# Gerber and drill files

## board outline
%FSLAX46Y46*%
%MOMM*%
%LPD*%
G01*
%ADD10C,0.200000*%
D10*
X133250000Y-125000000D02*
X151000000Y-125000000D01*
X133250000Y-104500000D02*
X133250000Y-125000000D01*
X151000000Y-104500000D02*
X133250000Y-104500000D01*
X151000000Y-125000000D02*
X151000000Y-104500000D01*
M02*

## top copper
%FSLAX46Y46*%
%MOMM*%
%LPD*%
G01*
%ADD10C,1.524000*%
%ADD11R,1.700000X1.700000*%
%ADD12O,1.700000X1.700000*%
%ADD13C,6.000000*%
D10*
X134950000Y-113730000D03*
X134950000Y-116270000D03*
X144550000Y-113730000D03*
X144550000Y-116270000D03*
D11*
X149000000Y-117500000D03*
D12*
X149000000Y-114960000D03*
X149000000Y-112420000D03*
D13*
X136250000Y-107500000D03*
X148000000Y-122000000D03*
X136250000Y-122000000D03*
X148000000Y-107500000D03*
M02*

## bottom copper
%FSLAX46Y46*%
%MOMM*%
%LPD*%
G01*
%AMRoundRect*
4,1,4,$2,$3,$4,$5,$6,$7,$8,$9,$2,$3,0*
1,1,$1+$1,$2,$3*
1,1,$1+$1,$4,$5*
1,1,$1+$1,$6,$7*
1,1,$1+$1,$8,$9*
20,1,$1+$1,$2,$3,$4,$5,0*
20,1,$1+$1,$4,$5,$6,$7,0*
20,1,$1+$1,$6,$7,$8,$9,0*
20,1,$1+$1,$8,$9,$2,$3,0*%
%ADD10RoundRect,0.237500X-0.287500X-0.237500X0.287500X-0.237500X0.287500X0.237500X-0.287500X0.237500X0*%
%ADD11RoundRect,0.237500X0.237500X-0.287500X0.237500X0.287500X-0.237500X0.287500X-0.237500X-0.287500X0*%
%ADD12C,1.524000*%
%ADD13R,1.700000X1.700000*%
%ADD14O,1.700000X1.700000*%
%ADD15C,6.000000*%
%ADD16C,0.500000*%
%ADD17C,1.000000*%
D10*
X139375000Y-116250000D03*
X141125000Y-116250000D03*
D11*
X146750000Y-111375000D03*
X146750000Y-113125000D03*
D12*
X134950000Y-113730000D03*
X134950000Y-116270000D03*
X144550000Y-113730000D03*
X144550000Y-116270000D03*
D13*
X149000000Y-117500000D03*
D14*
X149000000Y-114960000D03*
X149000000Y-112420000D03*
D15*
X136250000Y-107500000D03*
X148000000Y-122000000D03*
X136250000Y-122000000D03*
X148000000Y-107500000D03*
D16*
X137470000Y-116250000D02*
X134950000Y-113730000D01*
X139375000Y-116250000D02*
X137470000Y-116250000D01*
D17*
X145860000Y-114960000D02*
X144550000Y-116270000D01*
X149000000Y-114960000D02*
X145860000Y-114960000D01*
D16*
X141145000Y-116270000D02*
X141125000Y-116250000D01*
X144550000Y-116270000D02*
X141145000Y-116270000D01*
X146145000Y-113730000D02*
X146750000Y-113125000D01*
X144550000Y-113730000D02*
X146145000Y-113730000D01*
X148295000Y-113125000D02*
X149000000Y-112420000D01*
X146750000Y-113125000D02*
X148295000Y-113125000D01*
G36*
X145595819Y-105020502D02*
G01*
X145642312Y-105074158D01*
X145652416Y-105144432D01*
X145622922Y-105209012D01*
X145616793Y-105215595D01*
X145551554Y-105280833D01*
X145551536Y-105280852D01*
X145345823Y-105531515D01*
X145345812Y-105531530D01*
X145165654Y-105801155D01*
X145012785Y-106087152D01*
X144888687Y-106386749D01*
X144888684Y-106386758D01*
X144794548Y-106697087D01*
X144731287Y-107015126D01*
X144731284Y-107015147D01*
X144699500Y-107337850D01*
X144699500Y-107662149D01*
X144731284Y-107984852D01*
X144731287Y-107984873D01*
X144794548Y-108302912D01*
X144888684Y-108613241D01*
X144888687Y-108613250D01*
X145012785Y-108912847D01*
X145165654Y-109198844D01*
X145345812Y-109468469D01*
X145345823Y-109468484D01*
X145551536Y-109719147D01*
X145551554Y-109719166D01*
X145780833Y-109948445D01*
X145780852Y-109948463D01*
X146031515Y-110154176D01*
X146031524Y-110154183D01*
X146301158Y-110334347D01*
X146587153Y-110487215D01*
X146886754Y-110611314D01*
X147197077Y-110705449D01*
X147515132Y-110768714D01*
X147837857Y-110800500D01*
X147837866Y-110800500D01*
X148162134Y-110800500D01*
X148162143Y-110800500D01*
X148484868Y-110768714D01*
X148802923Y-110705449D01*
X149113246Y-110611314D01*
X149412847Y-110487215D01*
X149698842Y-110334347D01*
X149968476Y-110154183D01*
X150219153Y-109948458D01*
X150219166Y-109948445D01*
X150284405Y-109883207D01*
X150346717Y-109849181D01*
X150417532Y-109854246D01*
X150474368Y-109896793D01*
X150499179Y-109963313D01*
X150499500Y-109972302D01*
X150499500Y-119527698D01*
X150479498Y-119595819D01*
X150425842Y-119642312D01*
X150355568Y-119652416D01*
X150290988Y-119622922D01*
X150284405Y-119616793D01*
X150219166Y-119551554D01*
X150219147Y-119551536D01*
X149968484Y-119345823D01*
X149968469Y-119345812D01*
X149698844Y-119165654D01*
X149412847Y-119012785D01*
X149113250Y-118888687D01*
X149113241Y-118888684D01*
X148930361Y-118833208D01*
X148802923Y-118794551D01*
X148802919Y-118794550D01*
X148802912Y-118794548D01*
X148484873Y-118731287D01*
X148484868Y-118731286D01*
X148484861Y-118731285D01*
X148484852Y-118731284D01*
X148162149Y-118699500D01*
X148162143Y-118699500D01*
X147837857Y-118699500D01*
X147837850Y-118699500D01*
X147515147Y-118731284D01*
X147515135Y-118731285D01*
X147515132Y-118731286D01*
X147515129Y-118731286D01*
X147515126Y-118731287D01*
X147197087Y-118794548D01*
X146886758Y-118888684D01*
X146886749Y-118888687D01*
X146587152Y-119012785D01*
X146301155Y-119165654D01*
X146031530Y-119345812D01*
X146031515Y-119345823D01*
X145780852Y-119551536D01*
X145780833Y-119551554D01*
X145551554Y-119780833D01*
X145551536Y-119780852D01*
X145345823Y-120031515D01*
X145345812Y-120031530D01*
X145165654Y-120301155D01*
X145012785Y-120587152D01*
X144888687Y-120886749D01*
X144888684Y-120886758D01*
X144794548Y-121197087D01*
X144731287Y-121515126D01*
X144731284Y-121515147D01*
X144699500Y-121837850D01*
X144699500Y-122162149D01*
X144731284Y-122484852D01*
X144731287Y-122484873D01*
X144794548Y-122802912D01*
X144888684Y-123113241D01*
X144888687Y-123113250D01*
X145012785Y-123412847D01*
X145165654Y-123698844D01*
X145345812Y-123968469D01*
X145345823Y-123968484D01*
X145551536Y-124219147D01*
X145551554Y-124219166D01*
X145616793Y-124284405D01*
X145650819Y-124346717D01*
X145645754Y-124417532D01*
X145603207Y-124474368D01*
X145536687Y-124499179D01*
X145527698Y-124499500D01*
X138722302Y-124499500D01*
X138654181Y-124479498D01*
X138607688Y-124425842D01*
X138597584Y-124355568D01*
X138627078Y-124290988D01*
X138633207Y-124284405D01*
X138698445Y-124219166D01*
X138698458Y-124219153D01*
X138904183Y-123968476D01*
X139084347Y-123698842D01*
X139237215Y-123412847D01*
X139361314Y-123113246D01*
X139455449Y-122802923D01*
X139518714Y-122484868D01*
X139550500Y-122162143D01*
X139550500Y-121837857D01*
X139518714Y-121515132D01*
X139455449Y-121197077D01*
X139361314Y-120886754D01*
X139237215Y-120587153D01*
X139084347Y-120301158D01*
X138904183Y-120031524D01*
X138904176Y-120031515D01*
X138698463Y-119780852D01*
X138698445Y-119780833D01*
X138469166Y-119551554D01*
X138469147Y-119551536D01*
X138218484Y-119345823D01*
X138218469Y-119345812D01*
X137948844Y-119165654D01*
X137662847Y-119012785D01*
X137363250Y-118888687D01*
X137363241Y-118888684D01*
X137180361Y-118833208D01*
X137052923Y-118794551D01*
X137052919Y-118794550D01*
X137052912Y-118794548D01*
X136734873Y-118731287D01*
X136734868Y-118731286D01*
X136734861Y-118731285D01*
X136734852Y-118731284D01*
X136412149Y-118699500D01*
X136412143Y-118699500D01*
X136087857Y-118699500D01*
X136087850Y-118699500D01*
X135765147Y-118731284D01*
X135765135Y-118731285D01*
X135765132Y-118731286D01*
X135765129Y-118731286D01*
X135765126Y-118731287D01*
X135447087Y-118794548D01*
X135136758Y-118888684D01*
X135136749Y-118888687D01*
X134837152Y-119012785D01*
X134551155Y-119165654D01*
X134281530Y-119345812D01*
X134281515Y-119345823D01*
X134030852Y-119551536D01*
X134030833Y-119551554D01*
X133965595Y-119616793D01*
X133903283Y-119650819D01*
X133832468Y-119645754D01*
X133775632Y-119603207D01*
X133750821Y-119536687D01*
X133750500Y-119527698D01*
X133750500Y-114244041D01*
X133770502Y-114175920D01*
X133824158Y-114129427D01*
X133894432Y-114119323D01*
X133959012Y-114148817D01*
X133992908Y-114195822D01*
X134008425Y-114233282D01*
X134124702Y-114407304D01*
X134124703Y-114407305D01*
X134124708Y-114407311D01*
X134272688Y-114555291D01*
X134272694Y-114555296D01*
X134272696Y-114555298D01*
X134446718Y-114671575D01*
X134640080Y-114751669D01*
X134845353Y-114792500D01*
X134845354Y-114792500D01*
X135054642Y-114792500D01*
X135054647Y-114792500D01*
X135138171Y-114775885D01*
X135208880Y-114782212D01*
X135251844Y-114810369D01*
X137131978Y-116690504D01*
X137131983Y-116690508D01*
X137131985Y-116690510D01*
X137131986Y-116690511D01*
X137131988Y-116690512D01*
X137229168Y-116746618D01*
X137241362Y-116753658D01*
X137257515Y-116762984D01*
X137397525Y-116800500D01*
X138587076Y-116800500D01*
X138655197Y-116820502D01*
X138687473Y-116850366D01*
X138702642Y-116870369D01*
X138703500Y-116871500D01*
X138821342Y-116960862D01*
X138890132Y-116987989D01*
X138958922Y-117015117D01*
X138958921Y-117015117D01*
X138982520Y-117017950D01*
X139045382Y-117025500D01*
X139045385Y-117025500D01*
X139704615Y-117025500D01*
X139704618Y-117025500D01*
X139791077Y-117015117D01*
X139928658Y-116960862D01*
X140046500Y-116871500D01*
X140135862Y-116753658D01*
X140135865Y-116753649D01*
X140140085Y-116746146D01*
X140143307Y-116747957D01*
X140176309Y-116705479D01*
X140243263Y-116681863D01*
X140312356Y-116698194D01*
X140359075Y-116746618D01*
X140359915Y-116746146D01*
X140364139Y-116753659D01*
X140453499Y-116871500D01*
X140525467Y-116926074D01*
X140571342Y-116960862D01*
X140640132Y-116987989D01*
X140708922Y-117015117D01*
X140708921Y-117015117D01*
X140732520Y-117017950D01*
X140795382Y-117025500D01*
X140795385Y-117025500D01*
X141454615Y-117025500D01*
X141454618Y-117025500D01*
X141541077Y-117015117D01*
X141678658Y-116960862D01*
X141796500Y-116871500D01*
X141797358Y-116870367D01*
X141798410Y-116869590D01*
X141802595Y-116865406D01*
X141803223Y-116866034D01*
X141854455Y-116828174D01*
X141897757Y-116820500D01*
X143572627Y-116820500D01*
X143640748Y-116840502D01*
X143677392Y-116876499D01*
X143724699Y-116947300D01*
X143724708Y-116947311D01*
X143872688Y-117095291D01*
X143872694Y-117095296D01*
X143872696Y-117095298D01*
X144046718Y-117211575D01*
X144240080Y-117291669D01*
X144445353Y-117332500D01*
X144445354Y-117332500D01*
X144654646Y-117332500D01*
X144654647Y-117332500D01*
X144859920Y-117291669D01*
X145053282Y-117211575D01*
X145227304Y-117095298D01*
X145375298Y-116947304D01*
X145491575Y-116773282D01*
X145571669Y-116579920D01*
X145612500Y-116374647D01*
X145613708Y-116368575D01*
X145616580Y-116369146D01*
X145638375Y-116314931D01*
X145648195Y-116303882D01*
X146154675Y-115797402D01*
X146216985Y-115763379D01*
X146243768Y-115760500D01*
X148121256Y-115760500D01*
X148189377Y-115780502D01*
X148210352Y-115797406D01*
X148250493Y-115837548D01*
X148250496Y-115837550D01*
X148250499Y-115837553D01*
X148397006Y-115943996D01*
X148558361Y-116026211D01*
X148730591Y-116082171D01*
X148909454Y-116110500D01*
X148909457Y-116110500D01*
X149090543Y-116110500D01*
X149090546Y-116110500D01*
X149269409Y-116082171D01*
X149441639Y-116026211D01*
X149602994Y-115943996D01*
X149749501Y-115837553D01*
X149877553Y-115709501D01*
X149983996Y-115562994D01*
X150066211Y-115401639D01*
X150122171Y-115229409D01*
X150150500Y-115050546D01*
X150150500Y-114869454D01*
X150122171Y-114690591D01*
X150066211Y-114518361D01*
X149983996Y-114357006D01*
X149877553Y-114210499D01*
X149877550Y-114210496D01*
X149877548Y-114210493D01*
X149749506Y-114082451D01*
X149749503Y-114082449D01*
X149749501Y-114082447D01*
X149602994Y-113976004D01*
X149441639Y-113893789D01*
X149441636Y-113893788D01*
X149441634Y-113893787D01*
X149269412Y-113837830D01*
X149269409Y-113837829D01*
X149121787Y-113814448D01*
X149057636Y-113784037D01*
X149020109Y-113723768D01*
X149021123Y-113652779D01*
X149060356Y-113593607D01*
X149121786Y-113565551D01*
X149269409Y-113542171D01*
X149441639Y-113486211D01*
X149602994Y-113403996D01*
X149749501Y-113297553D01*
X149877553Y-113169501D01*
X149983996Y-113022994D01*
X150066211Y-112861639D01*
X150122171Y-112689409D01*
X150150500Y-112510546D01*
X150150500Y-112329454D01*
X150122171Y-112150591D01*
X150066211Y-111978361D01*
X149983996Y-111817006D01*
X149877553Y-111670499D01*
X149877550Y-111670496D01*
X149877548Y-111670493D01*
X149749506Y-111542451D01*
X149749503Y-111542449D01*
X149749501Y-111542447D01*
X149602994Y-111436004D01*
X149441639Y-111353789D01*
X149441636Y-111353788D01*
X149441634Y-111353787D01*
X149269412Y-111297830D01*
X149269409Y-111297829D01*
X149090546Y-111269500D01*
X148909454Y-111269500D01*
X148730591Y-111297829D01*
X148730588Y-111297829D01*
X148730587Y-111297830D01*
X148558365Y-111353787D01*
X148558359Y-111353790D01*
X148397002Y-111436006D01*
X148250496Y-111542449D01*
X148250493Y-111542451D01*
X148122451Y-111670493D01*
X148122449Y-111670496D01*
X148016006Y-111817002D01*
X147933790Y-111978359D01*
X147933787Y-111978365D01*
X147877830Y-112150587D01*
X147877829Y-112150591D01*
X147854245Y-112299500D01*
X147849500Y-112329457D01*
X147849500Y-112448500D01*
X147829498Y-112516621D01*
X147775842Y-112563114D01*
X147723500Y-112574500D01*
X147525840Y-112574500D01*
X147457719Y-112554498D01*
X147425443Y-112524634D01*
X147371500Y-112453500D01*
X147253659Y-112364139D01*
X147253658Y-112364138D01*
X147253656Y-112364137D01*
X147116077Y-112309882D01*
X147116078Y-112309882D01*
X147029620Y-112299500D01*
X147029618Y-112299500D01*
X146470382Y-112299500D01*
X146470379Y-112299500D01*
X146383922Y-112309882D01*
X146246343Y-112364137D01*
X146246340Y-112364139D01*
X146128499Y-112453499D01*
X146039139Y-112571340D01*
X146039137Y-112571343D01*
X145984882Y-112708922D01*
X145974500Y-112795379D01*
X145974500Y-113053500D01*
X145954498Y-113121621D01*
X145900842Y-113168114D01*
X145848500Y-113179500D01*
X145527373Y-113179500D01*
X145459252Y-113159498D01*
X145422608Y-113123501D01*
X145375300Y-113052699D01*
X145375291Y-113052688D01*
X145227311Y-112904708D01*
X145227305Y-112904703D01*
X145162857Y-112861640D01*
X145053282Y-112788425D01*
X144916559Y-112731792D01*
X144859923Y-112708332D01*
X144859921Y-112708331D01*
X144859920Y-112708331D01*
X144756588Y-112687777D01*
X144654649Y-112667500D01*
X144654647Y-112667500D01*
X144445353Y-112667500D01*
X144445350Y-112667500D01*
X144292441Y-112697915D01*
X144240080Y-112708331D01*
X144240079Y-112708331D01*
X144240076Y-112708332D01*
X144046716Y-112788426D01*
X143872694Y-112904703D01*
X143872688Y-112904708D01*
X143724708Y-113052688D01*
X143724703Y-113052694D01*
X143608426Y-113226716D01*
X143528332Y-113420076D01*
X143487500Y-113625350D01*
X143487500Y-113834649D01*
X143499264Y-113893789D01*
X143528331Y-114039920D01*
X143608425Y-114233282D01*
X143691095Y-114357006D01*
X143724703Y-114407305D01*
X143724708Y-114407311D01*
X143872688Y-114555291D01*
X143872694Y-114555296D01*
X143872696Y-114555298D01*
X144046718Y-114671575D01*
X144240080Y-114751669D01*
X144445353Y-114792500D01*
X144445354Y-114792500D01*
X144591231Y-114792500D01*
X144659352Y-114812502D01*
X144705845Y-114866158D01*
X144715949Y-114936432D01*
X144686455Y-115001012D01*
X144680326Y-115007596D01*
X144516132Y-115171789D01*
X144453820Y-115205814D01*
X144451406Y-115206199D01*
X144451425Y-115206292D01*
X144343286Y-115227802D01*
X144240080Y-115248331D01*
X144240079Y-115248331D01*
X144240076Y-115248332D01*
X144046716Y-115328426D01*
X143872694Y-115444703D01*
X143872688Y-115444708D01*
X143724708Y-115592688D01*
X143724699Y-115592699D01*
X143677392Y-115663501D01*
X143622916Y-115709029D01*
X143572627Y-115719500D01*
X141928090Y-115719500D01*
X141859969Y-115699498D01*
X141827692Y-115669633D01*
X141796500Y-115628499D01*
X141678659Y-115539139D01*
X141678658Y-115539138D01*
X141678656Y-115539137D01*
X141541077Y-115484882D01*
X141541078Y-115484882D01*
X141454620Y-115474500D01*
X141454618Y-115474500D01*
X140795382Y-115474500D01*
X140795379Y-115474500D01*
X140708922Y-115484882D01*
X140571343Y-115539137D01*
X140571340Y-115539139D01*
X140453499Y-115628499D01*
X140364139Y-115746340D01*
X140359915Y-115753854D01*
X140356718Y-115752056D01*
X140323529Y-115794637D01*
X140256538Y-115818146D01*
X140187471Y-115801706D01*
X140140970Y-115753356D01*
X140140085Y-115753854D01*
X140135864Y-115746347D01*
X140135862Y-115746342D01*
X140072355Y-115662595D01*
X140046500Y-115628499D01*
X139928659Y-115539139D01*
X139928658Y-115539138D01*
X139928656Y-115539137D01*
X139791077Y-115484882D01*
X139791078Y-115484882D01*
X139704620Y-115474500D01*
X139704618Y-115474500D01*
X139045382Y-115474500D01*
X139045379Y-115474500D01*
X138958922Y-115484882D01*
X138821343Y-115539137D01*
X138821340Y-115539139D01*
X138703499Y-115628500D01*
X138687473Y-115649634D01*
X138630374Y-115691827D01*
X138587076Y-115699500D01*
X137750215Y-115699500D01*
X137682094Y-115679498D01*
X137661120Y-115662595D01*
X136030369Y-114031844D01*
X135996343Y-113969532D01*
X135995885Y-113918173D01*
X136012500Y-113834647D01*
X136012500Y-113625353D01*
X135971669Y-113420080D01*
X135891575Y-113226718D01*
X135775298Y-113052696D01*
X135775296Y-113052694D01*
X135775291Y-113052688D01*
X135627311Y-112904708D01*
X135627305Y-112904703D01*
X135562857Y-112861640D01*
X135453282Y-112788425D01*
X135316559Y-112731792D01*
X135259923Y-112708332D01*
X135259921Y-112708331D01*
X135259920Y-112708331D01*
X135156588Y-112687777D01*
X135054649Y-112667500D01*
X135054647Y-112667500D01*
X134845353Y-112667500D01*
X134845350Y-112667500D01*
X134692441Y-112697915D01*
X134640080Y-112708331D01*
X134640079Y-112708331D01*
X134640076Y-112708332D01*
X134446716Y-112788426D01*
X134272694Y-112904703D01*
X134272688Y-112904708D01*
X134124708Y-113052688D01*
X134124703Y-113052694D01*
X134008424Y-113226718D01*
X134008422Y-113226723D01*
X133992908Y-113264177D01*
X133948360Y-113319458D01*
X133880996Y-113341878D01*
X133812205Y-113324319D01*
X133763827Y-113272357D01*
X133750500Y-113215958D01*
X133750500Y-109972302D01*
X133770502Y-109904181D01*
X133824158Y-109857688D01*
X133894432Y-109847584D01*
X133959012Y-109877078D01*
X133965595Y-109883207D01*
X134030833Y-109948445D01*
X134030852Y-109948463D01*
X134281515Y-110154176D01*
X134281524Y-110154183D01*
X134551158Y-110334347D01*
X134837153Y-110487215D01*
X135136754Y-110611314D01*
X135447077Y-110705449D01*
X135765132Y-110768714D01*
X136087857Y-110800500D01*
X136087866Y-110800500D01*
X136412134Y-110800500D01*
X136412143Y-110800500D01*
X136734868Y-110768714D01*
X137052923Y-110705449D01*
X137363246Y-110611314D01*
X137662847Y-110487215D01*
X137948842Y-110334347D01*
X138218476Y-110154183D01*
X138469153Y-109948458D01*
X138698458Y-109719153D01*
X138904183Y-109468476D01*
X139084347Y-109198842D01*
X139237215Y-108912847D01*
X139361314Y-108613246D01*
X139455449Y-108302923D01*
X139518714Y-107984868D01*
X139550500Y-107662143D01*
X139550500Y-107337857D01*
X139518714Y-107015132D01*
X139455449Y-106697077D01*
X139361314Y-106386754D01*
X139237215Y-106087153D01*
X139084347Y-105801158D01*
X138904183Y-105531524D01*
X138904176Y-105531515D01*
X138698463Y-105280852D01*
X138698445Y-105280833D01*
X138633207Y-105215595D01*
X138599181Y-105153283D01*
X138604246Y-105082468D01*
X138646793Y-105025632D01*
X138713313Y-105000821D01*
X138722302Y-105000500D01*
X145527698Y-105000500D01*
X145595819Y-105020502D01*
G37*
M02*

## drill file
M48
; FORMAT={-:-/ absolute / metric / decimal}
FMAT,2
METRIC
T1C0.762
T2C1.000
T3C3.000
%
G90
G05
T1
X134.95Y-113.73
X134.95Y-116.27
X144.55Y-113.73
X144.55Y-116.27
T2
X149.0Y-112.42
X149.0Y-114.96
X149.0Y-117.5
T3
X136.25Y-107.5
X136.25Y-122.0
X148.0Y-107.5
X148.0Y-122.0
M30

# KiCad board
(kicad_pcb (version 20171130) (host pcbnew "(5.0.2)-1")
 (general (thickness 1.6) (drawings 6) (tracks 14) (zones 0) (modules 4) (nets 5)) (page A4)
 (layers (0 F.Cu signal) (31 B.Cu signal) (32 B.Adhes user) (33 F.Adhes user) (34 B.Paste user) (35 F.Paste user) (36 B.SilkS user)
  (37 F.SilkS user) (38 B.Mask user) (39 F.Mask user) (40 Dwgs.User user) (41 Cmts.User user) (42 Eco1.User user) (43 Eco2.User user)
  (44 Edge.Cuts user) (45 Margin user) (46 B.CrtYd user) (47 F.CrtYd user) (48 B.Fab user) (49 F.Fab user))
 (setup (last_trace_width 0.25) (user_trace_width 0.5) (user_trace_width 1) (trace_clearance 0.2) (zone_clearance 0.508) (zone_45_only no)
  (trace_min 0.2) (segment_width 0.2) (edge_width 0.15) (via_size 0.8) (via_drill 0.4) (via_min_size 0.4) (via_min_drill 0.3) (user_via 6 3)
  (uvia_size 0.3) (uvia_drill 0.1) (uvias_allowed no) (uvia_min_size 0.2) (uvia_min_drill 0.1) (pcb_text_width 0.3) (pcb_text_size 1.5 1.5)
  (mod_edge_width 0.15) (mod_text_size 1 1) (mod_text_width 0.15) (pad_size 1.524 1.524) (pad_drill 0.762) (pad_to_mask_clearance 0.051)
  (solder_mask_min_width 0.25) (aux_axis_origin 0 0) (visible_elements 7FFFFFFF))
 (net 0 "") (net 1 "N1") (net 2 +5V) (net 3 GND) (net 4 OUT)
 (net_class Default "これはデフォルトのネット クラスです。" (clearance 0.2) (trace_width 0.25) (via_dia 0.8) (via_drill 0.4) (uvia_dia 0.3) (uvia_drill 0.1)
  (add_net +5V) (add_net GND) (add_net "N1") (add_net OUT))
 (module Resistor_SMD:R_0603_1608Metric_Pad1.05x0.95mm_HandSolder (layer B.Cu) (at 140.25 116.25)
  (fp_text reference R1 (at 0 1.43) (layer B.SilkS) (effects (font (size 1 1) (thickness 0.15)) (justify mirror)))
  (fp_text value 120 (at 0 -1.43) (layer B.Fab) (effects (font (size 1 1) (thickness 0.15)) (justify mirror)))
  (pad 1 smd roundrect (at -0.875 0) (size 1.05 0.95) (layers B.Cu B.Paste B.Mask) (roundrect_rratio 0.25) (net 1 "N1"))
  (pad 2 smd roundrect (at 0.875 0) (size 1.05 0.95) (layers B.Cu B.Paste B.Mask) (roundrect_rratio 0.25) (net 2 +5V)))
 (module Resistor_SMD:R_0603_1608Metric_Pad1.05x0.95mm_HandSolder (layer B.Cu) (at 146.75 112.25 90)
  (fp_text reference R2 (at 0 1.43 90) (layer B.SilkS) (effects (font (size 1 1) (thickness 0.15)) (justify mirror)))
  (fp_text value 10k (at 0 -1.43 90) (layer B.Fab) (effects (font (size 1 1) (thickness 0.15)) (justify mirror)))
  (pad 2 smd roundrect (at 0.875 0 90) (size 1.05 0.95) (layers B.Cu B.Paste B.Mask) (roundrect_rratio 0.25) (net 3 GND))
  (pad 1 smd roundrect (at -0.875 0 90) (size 1.05 0.95) (layers B.Cu B.Paste B.Mask) (roundrect_rratio 0.25) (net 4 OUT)))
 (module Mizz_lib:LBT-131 (layer F.Cu) (at 139.75 115)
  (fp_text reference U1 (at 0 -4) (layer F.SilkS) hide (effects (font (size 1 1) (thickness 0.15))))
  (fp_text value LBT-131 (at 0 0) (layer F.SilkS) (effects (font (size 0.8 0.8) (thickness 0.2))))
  (pad 1 thru_hole circle (at -4.8 -1.27) (size 1.524 1.524) (drill 0.762) (layers *.Cu *.Mask) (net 1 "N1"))
  (pad 2 thru_hole circle (at -4.8 1.27) (size 1.524 1.524) (drill 0.762) (layers *.Cu *.Mask) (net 3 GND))
  (pad 3 thru_hole circle (at 4.8 -1.27) (size 1.524 1.524) (drill 0.762) (layers *.Cu *.Mask) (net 4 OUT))
  (pad 4 thru_hole circle (at 4.8 1.27) (size 1.524 1.524) (drill 0.762) (layers *.Cu *.Mask) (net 2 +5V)))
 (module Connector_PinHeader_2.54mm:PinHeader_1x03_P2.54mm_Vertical (layer F.Cu) (at 149 117.5 180)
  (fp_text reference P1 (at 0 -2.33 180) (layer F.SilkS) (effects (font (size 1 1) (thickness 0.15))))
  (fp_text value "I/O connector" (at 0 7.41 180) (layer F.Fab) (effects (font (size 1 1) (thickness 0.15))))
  (pad 1 thru_hole rect (at 0 0 180) (size 1.7 1.7) (drill 1) (layers *.Cu *.Mask) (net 3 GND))
  (pad 2 thru_hole oval (at 0 2.54 180) (size 1.7 1.7) (drill 1) (layers *.Cu *.Mask) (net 2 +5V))
  (pad 3 thru_hole oval (at 0 5.08 180) (size 1.7 1.7) (drill 1) (layers *.Cu *.Mask) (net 4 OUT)))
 (gr_line (start 133.25 125) (end 151 125) (layer Edge.Cuts) (width 0.2))
 (gr_line (start 133.25 104.5) (end 133.25 125) (layer Edge.Cuts) (width 0.2))
 (gr_line (start 151 104.5) (end 133.25 104.5) (layer Edge.Cuts) (width 0.2))
 (gr_line (start 151 125) (end 151 104.5) (layer Edge.Cuts) (width 0.2))
 (via (at 136.25 107.5) (size 6) (drill 3) (layers F.Cu B.Cu) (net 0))
 (via (at 148 122) (size 6) (drill 3) (layers F.Cu B.Cu) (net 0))
 (via (at 136.25 122) (size 6) (drill 3) (layers F.Cu B.Cu) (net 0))
 (via (at 148 107.5) (size 6) (drill 3) (layers F.Cu B.Cu) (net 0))
 (segment (start 137.47 116.25) (end 134.95 113.73) (width 0.5) (layer B.Cu) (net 1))
 (segment (start 139.375 116.25) (end 137.47 116.25) (width 0.5) (layer B.Cu) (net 1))
 (segment (start 145.86 114.96) (end 144.55 116.27) (width 1) (layer B.Cu) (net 2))
 (segment (start 149 114.96) (end 145.86 114.96) (width 1) (layer B.Cu) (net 2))
 (segment (start 141.145 116.27) (end 141.125 116.25) (width 0.5) (layer B.Cu) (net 2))
 (segment (start 144.55 116.27) (end 141.145 116.27) (width 0.5) (layer B.Cu) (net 2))
 (segment (start 146.145 113.73) (end 146.75 113.125) (width 0.5) (layer B.Cu) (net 4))
 (segment (start 144.55 113.73) (end 146.145 113.73) (width 0.5) (layer B.Cu) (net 4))
 (segment (start 148.295 113.125) (end 149 112.42) (width 0.5) (layer B.Cu) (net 4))
 (segment (start 146.75 113.125) (end 148.295 113.125) (width 0.5) (layer B.Cu) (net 4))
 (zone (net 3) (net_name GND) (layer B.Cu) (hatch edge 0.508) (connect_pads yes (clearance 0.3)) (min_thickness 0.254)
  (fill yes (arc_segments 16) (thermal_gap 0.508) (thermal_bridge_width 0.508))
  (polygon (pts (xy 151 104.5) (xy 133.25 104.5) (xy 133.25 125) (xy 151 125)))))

